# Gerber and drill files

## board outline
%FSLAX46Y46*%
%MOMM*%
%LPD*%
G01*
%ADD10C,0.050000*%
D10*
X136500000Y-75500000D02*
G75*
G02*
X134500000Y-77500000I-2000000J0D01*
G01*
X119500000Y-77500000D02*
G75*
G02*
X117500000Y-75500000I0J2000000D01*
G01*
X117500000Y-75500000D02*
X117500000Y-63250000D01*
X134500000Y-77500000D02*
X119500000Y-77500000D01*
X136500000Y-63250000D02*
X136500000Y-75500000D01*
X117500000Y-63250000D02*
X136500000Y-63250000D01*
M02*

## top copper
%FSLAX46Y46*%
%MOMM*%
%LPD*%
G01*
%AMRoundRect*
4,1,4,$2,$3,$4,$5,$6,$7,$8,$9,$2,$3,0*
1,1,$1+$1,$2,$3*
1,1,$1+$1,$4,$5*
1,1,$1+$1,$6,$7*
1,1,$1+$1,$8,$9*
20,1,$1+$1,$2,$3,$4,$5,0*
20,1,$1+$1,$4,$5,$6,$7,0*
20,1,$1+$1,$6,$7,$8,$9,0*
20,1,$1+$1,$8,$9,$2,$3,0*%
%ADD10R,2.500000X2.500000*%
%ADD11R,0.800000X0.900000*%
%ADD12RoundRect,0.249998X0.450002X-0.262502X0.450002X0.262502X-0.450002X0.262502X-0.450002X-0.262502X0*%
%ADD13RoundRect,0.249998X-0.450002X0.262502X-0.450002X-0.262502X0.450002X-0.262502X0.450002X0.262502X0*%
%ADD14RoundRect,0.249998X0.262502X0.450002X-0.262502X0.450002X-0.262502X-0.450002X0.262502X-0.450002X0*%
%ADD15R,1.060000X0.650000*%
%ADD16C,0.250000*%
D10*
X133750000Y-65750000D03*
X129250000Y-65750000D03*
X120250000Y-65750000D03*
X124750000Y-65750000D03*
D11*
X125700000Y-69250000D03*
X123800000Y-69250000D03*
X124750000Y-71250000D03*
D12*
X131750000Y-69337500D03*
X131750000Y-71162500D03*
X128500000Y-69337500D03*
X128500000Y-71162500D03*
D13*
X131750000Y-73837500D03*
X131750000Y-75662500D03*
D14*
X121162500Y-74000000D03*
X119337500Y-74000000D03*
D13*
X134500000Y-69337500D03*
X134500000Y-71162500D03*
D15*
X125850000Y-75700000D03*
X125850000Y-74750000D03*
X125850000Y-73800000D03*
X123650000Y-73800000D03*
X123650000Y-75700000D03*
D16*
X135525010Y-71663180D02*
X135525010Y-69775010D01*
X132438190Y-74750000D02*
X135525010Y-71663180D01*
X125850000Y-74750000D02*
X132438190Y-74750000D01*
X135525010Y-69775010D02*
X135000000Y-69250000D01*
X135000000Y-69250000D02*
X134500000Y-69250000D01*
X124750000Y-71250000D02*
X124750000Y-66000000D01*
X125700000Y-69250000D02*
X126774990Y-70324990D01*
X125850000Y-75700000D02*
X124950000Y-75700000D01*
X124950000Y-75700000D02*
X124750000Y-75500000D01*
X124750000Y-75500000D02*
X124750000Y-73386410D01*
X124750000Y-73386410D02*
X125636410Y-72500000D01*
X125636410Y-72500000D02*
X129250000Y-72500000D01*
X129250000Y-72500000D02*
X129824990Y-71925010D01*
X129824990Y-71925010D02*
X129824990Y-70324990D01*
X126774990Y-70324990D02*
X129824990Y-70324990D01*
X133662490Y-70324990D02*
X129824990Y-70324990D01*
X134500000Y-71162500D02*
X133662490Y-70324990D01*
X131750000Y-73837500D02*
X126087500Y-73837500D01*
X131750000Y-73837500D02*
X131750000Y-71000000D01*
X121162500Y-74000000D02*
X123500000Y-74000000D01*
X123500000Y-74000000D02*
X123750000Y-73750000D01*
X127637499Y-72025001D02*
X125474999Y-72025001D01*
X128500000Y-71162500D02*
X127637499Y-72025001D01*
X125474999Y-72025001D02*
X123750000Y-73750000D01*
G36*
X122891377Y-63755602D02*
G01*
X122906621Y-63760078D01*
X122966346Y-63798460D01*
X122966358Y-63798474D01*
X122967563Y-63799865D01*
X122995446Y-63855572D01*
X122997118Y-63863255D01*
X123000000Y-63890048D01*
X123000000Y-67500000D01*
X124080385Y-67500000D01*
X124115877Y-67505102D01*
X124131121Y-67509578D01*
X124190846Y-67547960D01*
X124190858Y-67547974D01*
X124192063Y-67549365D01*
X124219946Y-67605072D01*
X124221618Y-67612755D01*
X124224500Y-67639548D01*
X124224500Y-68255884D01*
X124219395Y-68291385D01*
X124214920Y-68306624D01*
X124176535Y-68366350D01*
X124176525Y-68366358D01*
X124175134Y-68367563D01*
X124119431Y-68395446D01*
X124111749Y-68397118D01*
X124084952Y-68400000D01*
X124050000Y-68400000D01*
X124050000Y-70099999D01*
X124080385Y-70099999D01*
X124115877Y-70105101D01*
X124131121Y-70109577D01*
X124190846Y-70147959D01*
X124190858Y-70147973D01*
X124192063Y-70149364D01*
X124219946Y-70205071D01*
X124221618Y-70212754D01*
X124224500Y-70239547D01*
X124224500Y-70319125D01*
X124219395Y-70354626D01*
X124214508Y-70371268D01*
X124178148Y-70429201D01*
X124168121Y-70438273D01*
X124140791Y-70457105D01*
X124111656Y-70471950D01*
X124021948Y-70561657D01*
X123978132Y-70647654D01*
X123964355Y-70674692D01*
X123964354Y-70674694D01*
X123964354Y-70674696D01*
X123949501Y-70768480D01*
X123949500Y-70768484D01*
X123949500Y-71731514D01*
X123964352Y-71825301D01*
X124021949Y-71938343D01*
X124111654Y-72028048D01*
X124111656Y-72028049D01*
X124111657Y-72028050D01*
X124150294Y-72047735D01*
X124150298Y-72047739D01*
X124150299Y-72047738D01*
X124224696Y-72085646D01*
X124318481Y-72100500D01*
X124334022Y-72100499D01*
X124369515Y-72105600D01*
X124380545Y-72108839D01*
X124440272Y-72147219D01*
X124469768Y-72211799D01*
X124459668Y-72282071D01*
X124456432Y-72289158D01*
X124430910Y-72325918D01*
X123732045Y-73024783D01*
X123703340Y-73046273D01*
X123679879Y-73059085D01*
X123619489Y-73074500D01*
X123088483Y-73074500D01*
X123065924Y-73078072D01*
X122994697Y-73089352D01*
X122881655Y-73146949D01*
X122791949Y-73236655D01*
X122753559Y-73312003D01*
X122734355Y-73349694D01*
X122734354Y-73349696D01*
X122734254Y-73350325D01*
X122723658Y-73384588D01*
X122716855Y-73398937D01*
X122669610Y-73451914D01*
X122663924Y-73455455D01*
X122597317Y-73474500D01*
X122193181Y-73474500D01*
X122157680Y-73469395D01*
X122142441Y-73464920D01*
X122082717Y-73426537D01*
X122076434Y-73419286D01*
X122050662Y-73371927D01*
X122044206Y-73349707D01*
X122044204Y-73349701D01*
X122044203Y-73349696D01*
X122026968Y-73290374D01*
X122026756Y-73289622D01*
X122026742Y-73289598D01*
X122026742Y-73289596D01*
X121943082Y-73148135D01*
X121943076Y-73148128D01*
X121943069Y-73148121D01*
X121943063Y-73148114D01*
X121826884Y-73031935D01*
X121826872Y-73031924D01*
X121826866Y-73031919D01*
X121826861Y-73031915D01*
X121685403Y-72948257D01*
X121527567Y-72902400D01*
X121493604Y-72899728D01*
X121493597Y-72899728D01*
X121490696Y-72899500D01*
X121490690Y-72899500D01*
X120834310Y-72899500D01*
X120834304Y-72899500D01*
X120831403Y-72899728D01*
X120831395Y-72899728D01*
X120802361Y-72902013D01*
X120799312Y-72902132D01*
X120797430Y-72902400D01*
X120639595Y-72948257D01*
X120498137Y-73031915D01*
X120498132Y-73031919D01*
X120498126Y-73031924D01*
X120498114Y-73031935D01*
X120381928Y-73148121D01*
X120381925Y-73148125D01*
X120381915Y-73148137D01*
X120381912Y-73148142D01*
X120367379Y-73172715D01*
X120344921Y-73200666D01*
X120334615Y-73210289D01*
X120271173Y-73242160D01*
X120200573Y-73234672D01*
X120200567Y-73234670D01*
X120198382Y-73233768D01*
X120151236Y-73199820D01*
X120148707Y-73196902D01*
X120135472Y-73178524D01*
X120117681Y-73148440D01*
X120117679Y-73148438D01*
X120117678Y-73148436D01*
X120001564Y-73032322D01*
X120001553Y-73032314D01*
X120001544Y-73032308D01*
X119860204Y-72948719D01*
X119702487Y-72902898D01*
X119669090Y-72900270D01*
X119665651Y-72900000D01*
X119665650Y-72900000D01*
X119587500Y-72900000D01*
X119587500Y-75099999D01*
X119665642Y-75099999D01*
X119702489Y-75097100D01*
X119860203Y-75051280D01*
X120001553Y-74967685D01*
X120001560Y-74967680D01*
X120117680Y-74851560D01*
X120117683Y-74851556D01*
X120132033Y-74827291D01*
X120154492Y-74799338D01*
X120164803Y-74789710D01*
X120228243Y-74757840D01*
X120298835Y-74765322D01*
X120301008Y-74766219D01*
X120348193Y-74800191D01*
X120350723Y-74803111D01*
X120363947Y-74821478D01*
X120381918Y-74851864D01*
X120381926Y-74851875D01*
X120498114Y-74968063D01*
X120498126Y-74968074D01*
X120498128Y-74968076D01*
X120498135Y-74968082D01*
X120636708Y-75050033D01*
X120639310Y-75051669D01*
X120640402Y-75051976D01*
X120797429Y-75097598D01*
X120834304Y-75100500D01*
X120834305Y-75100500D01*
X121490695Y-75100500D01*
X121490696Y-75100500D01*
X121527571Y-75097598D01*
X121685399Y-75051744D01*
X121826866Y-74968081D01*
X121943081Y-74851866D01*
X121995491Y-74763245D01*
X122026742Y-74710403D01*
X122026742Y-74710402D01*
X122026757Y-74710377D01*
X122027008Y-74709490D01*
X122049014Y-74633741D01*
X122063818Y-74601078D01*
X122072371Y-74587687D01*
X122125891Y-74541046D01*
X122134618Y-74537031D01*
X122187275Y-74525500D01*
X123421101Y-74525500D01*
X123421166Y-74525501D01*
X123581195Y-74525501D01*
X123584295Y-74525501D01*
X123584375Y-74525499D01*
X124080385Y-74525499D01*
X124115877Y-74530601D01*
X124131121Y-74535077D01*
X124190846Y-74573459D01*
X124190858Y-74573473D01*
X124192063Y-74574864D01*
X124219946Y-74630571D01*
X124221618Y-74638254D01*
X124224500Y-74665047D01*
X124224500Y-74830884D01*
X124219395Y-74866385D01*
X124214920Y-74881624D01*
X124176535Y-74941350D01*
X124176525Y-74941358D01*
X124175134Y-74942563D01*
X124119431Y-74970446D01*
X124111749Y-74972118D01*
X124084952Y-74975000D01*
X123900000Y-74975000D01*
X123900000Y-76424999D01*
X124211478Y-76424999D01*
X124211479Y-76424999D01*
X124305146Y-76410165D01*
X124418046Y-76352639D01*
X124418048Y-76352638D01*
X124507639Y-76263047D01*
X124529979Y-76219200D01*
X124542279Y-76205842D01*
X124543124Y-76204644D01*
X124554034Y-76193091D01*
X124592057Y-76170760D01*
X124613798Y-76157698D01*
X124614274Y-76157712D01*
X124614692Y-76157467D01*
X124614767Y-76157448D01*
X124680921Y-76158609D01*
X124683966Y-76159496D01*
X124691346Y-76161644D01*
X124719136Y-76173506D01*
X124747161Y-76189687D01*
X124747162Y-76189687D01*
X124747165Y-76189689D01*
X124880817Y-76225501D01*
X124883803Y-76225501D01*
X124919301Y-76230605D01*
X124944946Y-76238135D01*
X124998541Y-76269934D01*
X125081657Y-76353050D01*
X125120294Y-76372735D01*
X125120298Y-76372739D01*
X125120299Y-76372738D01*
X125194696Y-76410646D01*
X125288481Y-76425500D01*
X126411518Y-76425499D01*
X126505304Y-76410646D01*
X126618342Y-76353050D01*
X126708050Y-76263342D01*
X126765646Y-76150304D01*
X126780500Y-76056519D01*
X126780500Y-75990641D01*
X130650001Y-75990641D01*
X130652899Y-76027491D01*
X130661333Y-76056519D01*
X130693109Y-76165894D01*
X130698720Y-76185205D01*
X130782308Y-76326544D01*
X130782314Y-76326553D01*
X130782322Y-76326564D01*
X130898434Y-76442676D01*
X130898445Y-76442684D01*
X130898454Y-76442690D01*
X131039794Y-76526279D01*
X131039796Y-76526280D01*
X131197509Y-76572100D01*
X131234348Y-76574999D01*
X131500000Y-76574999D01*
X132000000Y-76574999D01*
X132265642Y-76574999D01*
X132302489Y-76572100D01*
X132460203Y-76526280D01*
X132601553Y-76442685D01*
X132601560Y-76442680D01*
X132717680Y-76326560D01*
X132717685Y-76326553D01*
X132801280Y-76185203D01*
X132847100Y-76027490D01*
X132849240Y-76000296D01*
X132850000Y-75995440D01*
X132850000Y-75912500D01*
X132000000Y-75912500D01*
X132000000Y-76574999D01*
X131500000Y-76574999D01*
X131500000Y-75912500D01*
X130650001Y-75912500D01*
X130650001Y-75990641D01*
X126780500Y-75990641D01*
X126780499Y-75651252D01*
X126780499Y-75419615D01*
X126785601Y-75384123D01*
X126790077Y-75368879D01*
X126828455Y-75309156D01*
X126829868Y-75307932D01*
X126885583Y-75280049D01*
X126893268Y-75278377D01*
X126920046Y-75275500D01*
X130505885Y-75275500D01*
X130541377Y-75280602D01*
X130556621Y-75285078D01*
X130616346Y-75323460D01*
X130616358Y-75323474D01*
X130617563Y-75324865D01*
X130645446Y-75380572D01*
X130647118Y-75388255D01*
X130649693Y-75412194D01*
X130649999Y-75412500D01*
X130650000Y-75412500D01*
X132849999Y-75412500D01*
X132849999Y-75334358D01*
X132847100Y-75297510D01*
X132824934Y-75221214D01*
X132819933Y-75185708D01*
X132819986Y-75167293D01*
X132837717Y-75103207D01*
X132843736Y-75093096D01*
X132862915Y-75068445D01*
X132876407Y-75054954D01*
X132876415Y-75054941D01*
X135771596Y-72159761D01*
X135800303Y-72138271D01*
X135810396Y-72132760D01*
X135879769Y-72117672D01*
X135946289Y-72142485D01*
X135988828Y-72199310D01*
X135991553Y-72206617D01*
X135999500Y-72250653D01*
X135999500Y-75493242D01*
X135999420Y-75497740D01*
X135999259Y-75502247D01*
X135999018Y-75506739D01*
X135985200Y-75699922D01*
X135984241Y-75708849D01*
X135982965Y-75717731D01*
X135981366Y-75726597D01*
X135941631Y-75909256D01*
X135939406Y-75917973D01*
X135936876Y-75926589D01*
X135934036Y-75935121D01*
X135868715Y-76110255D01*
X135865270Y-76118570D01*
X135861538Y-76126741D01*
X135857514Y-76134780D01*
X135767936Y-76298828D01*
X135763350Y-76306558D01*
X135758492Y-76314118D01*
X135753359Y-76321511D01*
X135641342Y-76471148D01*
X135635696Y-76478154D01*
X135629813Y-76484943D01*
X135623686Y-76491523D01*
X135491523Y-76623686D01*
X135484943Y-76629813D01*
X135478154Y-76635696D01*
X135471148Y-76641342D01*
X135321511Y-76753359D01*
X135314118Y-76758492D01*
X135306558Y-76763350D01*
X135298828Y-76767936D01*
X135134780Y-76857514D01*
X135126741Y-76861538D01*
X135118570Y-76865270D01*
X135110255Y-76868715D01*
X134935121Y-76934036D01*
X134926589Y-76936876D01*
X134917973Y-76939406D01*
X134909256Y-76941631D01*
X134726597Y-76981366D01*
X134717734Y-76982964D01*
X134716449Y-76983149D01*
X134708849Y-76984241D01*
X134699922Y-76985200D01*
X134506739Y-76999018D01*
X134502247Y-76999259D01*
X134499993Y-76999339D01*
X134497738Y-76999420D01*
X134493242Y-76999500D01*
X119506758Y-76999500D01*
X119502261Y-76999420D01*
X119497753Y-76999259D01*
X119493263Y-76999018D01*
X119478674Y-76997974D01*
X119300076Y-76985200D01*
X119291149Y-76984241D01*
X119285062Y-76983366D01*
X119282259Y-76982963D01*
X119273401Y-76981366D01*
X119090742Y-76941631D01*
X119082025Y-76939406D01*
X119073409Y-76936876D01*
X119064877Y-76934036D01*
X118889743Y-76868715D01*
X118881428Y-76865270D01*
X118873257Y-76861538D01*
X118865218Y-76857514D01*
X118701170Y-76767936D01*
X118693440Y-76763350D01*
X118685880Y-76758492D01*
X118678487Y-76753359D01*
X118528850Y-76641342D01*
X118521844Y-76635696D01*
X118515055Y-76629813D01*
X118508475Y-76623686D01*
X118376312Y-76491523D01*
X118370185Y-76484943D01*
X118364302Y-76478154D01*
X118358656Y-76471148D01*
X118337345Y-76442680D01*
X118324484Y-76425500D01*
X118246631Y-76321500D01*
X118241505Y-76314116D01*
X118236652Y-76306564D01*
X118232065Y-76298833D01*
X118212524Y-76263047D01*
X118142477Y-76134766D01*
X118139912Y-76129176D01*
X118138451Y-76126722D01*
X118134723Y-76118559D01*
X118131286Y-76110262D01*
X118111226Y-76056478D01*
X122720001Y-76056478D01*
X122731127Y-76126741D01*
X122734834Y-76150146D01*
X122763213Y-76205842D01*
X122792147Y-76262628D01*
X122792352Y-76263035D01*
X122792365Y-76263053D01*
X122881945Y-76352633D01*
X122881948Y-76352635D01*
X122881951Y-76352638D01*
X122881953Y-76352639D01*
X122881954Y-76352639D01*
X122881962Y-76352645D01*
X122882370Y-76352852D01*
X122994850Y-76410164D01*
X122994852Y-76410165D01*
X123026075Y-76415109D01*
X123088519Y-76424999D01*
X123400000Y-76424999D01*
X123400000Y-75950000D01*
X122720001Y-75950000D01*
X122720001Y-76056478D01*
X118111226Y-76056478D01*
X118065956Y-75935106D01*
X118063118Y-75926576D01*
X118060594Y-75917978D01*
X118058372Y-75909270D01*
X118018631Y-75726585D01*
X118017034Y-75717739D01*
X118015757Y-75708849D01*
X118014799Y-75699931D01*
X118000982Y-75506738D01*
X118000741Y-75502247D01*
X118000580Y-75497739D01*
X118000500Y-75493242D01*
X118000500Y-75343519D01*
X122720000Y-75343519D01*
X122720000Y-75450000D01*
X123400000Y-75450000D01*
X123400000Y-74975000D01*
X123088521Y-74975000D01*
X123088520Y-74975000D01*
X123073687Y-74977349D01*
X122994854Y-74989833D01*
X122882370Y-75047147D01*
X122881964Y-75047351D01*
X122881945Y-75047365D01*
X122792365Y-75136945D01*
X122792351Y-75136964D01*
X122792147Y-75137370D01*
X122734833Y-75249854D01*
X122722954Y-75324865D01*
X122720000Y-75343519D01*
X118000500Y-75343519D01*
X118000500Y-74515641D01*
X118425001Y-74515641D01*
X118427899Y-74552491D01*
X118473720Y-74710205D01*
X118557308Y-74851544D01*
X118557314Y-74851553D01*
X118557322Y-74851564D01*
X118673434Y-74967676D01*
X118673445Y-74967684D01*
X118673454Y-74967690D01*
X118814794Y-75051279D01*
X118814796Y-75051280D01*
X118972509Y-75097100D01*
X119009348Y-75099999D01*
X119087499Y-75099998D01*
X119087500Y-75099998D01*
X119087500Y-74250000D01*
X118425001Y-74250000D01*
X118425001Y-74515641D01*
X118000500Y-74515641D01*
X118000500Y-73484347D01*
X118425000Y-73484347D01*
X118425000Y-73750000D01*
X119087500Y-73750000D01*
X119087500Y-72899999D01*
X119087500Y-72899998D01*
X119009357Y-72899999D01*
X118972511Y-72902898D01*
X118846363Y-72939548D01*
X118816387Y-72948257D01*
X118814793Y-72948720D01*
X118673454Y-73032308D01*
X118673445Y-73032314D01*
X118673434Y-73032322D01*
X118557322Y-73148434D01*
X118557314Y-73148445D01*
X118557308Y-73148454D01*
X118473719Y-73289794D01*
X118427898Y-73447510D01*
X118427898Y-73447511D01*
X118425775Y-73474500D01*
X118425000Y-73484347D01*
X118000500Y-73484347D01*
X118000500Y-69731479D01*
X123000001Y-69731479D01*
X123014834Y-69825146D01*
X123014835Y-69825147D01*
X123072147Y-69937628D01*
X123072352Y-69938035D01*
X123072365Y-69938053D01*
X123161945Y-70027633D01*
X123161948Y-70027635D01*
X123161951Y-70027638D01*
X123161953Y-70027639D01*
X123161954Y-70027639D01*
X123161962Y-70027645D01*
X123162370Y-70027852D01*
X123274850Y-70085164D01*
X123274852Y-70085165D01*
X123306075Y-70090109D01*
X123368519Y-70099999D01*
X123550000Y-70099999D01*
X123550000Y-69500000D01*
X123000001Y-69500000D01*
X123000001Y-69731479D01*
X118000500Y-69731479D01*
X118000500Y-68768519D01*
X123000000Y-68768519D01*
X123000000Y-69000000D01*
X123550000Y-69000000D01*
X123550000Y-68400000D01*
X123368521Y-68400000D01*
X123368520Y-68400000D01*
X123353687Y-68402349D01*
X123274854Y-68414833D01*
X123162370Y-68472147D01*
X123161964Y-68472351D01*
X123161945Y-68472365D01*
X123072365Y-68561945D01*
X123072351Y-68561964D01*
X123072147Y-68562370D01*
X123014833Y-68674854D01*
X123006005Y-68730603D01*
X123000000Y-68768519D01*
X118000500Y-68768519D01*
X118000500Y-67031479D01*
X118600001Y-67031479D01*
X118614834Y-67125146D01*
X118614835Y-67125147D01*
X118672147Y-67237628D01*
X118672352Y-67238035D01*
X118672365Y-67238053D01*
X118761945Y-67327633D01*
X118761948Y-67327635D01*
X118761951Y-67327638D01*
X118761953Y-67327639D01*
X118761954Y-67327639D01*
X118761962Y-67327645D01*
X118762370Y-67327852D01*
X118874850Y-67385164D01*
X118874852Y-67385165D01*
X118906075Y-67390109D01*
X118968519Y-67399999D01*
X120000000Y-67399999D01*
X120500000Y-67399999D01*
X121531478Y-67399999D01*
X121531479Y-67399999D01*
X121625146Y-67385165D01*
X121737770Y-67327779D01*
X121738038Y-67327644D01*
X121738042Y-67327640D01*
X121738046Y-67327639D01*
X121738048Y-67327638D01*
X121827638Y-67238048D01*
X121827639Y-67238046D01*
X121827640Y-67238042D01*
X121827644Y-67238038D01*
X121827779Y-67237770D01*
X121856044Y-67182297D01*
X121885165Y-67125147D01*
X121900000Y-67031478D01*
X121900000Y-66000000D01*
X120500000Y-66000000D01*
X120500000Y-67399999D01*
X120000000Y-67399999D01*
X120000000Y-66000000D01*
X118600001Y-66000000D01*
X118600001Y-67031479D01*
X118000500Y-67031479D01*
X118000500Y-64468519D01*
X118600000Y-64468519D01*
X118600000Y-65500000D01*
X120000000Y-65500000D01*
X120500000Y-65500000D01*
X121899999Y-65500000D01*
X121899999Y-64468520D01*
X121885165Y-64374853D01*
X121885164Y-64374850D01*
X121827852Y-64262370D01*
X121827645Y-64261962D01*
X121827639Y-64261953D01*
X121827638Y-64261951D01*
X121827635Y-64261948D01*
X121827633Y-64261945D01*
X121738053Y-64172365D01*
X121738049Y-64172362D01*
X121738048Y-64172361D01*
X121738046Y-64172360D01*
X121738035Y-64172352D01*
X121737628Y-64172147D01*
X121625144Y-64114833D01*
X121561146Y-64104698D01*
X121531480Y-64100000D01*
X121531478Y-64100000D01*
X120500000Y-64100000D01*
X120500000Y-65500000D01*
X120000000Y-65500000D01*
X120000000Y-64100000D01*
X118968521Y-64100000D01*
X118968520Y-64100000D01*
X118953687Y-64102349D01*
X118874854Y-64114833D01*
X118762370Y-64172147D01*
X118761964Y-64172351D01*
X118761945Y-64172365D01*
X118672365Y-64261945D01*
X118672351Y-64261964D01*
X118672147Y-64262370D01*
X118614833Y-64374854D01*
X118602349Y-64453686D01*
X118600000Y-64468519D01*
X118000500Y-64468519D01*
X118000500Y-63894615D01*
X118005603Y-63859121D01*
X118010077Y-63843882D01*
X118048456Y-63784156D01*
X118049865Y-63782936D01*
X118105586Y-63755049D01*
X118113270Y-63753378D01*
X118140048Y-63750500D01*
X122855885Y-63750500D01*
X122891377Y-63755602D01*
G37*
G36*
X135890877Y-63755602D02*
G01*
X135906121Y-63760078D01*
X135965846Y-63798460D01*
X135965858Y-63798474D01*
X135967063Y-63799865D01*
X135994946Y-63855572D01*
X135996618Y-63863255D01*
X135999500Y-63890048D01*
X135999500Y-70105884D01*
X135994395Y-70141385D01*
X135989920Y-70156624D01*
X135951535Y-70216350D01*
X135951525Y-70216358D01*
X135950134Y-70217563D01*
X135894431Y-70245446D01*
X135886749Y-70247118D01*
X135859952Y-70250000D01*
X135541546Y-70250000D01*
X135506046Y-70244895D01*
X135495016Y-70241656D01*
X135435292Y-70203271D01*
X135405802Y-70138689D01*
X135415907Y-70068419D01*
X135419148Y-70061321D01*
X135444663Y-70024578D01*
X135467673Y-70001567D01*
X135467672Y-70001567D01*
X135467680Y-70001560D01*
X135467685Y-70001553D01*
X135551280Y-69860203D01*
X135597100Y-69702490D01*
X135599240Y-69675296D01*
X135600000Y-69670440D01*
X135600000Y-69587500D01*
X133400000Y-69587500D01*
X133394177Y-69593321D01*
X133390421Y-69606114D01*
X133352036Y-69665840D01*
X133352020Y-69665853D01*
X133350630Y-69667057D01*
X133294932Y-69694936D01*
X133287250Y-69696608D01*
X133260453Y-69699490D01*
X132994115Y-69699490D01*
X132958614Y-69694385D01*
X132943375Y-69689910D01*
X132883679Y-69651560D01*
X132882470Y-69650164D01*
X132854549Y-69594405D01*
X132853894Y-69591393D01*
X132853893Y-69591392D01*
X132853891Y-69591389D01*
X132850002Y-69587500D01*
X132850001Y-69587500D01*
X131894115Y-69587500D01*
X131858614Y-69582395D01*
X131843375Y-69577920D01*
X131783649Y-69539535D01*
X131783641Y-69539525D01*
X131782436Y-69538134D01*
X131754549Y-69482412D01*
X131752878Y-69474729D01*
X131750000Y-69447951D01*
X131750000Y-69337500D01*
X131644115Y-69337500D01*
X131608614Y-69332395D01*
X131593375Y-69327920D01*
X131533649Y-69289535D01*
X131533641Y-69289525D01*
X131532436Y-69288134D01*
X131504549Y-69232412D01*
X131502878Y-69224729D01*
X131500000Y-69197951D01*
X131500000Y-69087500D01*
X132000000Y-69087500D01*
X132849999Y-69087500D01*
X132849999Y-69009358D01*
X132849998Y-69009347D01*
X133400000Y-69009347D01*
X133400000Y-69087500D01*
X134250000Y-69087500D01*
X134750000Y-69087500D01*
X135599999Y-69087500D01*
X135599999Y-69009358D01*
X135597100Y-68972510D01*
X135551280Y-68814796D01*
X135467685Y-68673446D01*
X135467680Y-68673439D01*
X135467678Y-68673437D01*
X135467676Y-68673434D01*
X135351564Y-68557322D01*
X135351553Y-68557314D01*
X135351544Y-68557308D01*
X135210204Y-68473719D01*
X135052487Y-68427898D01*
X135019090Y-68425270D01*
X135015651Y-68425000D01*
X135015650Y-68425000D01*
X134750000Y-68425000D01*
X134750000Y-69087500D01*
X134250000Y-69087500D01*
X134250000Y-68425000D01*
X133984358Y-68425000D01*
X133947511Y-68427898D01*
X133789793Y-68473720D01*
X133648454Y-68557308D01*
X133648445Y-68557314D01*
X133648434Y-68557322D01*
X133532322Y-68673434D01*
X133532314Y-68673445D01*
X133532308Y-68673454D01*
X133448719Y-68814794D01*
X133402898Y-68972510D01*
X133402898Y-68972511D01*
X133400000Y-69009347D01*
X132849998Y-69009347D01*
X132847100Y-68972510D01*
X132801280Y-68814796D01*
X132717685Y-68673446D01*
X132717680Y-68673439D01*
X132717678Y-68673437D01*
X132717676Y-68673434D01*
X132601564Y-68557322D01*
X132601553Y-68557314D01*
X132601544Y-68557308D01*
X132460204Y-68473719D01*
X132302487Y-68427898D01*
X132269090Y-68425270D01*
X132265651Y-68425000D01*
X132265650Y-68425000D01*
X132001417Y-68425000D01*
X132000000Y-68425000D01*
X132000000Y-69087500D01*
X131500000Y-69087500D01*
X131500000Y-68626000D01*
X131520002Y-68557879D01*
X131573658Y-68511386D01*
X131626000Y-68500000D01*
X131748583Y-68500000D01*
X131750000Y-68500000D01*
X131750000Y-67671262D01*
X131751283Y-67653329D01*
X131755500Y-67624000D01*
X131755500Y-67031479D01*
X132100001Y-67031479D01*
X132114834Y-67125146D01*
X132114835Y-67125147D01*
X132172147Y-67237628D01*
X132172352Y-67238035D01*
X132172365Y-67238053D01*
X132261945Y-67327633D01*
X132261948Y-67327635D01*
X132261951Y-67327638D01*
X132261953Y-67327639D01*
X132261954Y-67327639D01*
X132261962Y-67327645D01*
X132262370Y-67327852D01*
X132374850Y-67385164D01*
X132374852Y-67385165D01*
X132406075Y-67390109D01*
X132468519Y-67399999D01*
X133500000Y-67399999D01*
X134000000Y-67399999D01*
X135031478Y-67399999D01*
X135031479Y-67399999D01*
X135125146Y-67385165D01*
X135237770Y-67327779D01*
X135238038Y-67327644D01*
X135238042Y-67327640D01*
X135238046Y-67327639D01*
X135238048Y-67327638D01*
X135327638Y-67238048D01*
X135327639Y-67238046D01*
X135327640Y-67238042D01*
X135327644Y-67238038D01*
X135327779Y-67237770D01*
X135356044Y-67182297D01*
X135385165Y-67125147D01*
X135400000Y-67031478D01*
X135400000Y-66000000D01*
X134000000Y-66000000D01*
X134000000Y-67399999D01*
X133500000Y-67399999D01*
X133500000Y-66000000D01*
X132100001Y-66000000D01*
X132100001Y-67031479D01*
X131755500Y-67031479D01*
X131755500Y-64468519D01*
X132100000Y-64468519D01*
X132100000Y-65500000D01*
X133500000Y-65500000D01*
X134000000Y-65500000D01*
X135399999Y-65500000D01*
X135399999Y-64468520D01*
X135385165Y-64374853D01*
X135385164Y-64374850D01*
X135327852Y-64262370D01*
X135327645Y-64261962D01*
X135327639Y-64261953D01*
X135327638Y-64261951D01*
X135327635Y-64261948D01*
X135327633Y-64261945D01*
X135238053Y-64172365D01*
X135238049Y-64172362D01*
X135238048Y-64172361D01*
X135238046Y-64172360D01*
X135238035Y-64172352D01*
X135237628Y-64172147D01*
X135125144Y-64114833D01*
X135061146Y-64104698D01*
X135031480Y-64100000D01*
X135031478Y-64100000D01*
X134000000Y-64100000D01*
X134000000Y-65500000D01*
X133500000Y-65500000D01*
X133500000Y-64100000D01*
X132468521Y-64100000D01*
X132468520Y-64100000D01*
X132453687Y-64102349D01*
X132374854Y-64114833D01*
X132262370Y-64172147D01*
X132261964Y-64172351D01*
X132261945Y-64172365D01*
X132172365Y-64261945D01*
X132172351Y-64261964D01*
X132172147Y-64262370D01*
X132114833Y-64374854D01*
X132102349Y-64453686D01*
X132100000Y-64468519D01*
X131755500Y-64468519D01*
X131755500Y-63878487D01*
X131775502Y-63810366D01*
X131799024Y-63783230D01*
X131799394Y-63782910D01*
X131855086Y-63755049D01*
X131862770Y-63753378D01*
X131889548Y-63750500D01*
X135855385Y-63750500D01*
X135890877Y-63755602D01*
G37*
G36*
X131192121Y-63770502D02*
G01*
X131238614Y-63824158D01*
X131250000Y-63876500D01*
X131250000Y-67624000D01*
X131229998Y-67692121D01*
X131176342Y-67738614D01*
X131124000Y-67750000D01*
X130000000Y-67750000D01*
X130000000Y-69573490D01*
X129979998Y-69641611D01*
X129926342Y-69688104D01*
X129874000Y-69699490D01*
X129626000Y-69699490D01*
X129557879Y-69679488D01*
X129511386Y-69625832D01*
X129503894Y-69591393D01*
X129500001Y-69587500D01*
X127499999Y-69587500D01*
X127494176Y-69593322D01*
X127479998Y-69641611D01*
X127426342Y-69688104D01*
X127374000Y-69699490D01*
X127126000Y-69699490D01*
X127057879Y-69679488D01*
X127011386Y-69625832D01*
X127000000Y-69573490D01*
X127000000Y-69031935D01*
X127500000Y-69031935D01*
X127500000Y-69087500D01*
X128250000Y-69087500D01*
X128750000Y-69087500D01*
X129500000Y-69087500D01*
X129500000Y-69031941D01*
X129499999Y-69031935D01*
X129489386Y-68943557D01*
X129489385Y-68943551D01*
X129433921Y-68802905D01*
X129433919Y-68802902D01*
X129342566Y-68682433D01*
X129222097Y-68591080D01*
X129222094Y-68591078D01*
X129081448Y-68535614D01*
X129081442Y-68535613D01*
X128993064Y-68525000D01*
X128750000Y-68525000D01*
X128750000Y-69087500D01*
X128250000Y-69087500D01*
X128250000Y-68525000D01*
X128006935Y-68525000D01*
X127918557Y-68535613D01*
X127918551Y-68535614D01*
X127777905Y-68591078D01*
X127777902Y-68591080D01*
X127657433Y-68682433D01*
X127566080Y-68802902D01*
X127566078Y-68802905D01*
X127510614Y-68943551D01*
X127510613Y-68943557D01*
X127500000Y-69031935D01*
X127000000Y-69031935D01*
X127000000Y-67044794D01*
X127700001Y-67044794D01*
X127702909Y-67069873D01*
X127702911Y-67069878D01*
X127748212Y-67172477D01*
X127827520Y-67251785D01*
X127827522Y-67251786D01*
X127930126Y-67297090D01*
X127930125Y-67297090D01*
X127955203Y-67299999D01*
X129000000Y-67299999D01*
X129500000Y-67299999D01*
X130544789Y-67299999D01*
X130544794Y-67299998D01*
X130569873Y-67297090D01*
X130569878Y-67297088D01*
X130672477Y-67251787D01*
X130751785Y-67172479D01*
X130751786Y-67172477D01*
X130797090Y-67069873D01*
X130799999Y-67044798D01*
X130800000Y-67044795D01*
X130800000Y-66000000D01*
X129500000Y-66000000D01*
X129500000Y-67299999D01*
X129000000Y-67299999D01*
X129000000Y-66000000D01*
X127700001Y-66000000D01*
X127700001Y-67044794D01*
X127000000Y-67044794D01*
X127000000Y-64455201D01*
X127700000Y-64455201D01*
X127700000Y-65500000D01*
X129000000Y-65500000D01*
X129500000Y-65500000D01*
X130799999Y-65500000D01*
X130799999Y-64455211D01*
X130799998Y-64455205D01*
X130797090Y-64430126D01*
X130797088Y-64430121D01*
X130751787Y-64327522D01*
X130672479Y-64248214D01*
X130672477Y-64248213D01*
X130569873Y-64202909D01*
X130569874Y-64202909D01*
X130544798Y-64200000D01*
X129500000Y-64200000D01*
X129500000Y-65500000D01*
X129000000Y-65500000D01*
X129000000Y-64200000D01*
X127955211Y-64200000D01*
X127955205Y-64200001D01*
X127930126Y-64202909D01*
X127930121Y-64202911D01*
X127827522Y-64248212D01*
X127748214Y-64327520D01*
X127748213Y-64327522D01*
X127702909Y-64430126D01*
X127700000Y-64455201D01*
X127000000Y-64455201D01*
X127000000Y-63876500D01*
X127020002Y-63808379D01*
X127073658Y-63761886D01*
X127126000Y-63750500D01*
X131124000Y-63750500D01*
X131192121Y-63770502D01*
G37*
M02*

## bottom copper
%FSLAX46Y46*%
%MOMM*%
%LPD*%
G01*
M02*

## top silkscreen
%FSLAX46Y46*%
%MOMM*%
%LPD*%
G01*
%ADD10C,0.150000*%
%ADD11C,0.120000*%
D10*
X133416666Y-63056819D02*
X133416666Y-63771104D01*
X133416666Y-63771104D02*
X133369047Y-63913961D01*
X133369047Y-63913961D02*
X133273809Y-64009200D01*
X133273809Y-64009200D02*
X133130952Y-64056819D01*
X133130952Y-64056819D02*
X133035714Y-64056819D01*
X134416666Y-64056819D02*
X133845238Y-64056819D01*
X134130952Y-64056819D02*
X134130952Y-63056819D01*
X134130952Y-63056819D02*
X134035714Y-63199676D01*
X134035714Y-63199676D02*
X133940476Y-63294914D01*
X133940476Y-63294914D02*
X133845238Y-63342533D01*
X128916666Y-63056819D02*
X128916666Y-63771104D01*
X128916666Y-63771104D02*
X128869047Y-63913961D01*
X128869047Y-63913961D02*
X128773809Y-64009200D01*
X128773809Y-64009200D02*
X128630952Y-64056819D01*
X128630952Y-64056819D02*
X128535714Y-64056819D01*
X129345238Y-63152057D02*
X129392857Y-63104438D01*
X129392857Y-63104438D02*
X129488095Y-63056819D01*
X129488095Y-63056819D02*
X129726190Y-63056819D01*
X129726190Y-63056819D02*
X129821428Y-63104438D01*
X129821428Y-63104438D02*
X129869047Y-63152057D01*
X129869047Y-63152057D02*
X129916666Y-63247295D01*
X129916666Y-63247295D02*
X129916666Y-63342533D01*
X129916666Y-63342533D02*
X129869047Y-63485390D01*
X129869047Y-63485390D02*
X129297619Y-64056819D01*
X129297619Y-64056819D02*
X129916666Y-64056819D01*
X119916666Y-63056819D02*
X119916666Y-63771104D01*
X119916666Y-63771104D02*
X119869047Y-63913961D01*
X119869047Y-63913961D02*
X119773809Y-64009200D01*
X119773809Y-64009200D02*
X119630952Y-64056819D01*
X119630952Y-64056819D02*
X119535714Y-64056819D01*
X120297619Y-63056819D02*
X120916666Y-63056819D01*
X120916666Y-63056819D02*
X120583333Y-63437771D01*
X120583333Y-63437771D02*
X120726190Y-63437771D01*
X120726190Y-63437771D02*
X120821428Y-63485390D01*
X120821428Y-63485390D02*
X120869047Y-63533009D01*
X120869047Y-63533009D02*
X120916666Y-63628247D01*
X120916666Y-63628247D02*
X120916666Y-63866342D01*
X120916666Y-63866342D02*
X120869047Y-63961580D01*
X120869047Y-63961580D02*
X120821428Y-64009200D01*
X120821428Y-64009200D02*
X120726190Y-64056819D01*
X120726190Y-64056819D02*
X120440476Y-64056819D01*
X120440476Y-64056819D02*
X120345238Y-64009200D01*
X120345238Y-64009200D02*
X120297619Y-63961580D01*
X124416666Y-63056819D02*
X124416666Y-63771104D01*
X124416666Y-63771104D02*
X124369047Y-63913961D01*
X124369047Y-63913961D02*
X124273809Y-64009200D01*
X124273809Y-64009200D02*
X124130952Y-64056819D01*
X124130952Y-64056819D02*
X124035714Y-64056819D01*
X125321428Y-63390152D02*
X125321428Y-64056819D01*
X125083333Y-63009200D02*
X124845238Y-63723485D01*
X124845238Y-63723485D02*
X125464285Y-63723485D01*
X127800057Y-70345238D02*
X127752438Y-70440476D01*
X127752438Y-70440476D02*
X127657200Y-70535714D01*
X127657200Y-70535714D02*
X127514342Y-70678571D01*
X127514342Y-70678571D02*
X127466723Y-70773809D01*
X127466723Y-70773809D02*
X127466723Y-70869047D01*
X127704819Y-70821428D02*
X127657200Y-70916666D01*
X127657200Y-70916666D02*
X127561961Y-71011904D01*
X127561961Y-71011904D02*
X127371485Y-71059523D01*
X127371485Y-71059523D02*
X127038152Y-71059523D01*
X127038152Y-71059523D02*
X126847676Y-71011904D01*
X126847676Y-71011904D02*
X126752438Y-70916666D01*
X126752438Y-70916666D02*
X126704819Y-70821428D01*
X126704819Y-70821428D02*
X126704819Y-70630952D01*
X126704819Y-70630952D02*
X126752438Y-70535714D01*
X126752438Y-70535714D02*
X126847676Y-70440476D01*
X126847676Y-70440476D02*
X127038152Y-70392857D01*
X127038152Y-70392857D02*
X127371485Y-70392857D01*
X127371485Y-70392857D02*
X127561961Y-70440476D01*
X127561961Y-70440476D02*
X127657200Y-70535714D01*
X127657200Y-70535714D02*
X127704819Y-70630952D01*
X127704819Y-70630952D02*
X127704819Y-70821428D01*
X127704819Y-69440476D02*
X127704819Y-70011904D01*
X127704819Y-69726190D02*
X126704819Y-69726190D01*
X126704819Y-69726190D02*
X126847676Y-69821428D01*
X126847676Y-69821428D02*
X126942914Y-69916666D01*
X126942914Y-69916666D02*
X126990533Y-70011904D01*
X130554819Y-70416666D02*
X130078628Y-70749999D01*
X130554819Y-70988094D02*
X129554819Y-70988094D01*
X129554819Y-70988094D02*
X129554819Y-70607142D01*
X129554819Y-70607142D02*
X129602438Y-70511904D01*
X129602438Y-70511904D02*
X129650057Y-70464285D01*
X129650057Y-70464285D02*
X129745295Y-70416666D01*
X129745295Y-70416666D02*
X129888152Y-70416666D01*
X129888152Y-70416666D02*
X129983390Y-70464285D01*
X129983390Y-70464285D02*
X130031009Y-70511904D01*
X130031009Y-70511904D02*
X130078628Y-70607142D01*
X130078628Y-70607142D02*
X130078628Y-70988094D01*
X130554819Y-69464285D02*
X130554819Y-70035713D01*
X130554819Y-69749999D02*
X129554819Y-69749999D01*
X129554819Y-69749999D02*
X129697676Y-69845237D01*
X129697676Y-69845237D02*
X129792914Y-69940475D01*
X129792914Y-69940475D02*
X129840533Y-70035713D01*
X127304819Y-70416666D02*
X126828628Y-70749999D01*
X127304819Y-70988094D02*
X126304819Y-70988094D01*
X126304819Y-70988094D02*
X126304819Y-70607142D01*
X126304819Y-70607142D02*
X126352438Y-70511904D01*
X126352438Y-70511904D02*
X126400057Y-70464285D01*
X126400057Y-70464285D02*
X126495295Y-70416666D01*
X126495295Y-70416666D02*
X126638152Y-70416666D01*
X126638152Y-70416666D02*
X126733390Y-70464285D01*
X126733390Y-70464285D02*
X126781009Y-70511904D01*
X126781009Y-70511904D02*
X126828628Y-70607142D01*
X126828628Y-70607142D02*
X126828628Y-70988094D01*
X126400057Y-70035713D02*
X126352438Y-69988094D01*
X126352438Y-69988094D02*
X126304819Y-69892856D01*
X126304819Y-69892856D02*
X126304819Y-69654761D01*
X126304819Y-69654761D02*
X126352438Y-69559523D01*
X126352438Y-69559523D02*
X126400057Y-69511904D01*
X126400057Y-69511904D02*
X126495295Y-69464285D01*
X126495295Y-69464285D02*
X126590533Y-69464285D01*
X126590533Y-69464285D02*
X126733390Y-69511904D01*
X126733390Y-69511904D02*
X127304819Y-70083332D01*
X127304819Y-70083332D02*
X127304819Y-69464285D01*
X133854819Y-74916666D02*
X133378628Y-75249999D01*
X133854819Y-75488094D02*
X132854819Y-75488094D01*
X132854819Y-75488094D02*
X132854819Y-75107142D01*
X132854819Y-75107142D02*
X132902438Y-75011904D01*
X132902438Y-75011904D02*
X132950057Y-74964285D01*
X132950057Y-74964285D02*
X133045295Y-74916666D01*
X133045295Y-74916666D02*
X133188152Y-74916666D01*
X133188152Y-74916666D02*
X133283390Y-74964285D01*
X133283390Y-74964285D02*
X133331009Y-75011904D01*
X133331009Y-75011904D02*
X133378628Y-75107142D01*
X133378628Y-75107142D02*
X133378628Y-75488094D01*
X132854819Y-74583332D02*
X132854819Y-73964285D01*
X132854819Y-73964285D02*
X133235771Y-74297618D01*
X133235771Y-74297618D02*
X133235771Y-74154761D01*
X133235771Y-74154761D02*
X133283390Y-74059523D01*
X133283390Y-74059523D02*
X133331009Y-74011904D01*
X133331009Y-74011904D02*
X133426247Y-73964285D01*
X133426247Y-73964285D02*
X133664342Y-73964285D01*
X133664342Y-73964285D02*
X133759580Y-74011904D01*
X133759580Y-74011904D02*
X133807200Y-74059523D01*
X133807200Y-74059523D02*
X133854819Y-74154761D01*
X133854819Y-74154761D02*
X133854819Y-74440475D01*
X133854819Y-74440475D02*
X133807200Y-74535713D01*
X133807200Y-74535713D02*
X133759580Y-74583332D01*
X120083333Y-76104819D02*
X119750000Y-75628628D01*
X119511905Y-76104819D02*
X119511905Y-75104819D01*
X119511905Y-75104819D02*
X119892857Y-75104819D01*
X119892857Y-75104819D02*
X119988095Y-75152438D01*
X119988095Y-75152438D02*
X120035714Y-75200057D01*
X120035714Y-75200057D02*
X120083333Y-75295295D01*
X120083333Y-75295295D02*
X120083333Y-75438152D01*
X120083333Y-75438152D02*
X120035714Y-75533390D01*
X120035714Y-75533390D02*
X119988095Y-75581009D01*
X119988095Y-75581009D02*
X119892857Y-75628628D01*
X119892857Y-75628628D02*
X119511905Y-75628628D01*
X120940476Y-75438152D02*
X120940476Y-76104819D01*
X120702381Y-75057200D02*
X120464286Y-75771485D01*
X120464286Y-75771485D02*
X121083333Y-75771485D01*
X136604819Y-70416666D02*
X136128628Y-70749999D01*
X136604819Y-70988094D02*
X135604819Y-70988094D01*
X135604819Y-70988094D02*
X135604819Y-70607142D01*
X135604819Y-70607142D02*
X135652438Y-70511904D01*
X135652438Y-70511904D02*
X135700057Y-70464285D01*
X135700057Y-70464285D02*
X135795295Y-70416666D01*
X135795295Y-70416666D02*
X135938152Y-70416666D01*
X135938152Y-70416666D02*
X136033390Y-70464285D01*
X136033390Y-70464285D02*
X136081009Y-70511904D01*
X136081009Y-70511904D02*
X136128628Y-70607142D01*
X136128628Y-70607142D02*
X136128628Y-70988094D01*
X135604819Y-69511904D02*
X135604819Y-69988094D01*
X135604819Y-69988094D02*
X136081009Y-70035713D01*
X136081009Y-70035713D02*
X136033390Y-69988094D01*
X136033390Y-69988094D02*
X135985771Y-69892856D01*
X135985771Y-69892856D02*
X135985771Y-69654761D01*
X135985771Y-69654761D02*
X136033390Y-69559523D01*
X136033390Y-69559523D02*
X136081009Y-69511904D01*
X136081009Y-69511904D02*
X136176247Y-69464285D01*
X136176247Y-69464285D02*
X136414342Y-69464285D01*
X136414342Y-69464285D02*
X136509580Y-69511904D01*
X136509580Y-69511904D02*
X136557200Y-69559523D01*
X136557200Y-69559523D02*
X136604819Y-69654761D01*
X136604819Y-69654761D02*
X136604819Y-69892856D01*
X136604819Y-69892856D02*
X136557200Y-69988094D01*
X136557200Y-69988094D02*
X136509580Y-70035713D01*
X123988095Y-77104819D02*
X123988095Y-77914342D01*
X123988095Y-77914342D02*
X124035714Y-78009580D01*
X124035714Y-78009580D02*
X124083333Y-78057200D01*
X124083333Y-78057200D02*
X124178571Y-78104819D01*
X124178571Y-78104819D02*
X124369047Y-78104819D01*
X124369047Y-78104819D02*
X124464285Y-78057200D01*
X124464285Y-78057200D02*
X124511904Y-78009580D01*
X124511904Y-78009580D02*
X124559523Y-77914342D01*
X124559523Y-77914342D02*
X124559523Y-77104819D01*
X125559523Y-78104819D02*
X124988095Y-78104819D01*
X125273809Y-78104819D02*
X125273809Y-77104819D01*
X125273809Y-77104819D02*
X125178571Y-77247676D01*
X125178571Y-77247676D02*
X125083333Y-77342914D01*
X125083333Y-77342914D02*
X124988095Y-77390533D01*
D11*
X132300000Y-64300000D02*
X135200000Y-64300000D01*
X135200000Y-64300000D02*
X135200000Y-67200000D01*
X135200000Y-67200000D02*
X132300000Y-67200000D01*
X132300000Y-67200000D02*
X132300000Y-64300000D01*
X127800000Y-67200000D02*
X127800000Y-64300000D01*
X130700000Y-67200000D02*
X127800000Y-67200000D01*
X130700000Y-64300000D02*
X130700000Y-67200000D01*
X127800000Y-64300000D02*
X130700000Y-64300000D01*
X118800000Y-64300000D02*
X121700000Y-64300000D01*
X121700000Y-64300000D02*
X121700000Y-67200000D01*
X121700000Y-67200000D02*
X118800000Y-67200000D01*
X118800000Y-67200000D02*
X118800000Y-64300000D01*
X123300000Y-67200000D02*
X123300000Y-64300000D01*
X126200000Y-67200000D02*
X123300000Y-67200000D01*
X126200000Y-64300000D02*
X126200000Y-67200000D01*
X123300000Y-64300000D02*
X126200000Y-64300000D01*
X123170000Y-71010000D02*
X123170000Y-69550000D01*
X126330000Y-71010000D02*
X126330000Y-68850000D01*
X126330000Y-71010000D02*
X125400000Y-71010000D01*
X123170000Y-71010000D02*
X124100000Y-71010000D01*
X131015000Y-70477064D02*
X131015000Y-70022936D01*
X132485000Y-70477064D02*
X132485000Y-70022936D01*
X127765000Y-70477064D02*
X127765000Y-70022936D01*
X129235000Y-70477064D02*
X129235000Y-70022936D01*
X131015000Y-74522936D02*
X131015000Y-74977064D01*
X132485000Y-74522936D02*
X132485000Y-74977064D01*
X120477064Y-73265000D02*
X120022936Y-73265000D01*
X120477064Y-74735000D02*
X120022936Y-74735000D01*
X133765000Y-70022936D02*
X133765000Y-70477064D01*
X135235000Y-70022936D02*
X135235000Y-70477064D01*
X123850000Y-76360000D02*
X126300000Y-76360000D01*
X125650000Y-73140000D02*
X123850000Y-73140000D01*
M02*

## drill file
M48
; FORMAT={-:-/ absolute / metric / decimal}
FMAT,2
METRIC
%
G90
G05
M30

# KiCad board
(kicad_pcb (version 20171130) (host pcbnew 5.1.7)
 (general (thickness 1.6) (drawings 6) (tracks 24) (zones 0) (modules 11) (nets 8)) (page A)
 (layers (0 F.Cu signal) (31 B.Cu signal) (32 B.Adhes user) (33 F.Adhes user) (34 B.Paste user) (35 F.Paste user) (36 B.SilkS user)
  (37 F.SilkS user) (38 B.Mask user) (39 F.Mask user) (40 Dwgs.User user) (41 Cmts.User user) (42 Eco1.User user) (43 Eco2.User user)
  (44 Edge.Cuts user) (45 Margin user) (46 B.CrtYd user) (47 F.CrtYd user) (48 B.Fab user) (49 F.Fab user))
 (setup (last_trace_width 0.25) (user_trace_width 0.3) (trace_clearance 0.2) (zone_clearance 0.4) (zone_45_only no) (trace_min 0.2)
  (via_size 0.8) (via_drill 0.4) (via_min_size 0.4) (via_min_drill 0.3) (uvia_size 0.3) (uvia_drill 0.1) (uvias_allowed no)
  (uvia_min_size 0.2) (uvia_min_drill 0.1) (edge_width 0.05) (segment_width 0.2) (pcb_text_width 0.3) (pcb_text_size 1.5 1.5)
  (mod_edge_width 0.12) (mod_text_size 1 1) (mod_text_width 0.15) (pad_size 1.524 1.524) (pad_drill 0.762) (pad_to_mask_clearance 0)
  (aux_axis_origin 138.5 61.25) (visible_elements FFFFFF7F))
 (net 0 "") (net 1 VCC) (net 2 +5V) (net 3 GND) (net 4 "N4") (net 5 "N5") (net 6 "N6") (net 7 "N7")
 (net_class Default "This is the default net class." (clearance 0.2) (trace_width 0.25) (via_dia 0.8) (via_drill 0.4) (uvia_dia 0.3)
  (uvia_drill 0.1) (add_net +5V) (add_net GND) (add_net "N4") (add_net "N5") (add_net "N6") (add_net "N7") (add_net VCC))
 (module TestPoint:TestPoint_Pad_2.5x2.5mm (layer F.Cu) (at 133.75 65.75)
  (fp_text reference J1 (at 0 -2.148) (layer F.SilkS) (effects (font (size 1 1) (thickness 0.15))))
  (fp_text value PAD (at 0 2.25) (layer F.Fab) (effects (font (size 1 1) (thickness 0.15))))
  (fp_line (start -1.45 -1.45) (end 1.45 -1.45) (layer F.SilkS) (width 0.12))
  (fp_line (start 1.45 -1.45) (end 1.45 1.45) (layer F.SilkS) (width 0.12))
  (fp_line (start 1.45 1.45) (end -1.45 1.45) (layer F.SilkS) (width 0.12))
  (fp_line (start -1.45 1.45) (end -1.45 -1.45) (layer F.SilkS) (width 0.12))
  (pad 1 smd rect (at 0 0) (size 2.5 2.5) (layers F.Cu F.Mask) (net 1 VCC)))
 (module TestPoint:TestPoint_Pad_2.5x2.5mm (layer F.Cu) (at 129.25 65.75)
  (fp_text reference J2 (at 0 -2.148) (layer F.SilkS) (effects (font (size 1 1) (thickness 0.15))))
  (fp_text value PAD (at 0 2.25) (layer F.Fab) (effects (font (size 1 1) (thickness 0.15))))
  (fp_line (start -1.45 1.45) (end -1.45 -1.45) (layer F.SilkS) (width 0.12))
  (fp_line (start 1.45 1.45) (end -1.45 1.45) (layer F.SilkS) (width 0.12))
  (fp_line (start 1.45 -1.45) (end 1.45 1.45) (layer F.SilkS) (width 0.12))
  (fp_line (start -1.45 -1.45) (end 1.45 -1.45) (layer F.SilkS) (width 0.12))
  (pad 1 smd rect (at 0 0) (size 2.5 2.5) (layers F.Cu F.Mask) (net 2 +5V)))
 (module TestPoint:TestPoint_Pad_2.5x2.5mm (layer F.Cu) (at 120.25 65.75)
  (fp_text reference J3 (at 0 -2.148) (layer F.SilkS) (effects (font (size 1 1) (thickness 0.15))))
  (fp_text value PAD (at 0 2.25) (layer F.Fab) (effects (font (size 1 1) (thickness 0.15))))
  (fp_line (start -1.45 -1.45) (end 1.45 -1.45) (layer F.SilkS) (width 0.12))
  (fp_line (start 1.45 -1.45) (end 1.45 1.45) (layer F.SilkS) (width 0.12))
  (fp_line (start 1.45 1.45) (end -1.45 1.45) (layer F.SilkS) (width 0.12))
  (fp_line (start -1.45 1.45) (end -1.45 -1.45) (layer F.SilkS) (width 0.12))
  (pad 1 smd rect (at 0 0) (size 2.5 2.5) (layers F.Cu F.Mask) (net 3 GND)))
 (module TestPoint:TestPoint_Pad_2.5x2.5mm (layer F.Cu) (at 124.75 65.75)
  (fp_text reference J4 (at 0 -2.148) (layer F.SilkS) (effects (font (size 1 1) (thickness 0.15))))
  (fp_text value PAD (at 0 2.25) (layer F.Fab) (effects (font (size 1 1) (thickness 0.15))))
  (fp_line (start -1.45 1.45) (end -1.45 -1.45) (layer F.SilkS) (width 0.12))
  (fp_line (start 1.45 1.45) (end -1.45 1.45) (layer F.SilkS) (width 0.12))
  (fp_line (start 1.45 -1.45) (end 1.45 1.45) (layer F.SilkS) (width 0.12))
  (fp_line (start -1.45 -1.45) (end 1.45 -1.45) (layer F.SilkS) (width 0.12))
  (pad 1 smd rect (at 0 0) (size 2.5 2.5) (layers F.Cu F.Mask) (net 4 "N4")))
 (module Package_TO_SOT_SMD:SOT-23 (layer F.Cu) (at 124.75 70.25 270)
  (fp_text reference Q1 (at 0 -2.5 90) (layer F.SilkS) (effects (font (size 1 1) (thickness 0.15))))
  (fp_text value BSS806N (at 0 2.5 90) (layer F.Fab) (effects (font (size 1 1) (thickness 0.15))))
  (fp_line (start 0.76 1.58) (end -0.7 1.58) (layer F.SilkS) (width 0.12))
  (fp_line (start 0.76 -1.58) (end -1.4 -1.58) (layer F.SilkS) (width 0.12))
  (fp_line (start 0.76 -1.58) (end 0.76 -0.65) (layer F.SilkS) (width 0.12))
  (fp_line (start 0.76 1.58) (end 0.76 0.65) (layer F.SilkS) (width 0.12))
  (pad 1 smd rect (at -1 -0.95 270) (size 0.9 0.8) (layers F.Cu F.Paste F.Mask) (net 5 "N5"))
  (pad 2 smd rect (at -1 0.95 270) (size 0.9 0.8) (layers F.Cu F.Paste F.Mask) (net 3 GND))
  (pad 3 smd rect (at 1 0 270) (size 0.9 0.8) (layers F.Cu F.Paste F.Mask) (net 4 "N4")))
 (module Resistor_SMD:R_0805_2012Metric (layer F.Cu) (at 131.75 70.25 90)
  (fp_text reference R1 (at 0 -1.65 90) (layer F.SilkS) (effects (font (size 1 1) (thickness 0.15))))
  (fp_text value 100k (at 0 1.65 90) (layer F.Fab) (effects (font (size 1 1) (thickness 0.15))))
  (fp_line (start -0.227064 -0.735) (end 0.227064 -0.735) (layer F.SilkS) (width 0.12))
  (fp_line (start -0.227064 0.735) (end 0.227064 0.735) (layer F.SilkS) (width 0.12))
  (pad 2 smd roundrect (at 0.9125 0 90) (size 1.025 1.4) (layers F.Cu F.Paste F.Mask) (roundrect_rratio 0.2439004878048781) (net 1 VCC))
  (pad 1 smd roundrect (at -0.9125 0 90) (size 1.025 1.4) (layers F.Cu F.Paste F.Mask) (roundrect_rratio 0.2439004878048781) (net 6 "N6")))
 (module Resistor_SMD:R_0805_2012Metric (layer F.Cu) (at 128.5 70.25 90)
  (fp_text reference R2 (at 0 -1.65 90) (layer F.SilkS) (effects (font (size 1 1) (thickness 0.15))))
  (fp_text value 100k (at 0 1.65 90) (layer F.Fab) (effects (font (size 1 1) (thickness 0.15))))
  (fp_line (start -0.227064 -0.735) (end 0.227064 -0.735) (layer F.SilkS) (width 0.12))
  (fp_line (start -0.227064 0.735) (end 0.227064 0.735) (layer F.SilkS) (width 0.12))
  (pad 2 smd roundrect (at 0.9125 0 90) (size 1.025 1.4) (layers F.Cu F.Paste F.Mask) (roundrect_rratio 0.2439004878048781) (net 2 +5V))
  (pad 1 smd roundrect (at -0.9125 0 90) (size 1.025 1.4) (layers F.Cu F.Paste F.Mask) (roundrect_rratio 0.2439004878048781) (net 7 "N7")))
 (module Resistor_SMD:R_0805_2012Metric (layer F.Cu) (at 131.75 74.75 270)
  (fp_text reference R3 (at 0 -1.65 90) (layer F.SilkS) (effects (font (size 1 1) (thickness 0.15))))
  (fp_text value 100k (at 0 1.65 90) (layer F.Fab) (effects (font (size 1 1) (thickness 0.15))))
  (fp_line (start -0.227064 0.735) (end 0.227064 0.735) (layer F.SilkS) (width 0.12))
  (fp_line (start -0.227064 -0.735) (end 0.227064 -0.735) (layer F.SilkS) (width 0.12))
  (pad 1 smd roundrect (at -0.9125 0 270) (size 1.025 1.4) (layers F.Cu F.Paste F.Mask) (roundrect_rratio 0.2439004878048781) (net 6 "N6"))
  (pad 2 smd roundrect (at 0.9125 0 270) (size 1.025 1.4) (layers F.Cu F.Paste F.Mask) (roundrect_rratio 0.2439004878048781) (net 3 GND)))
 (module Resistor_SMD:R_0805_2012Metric (layer F.Cu) (at 120.25 74 180)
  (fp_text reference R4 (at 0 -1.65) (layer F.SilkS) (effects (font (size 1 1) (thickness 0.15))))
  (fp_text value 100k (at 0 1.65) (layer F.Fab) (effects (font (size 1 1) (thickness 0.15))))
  (fp_line (start -0.227064 0.735) (end 0.227064 0.735) (layer F.SilkS) (width 0.12))
  (fp_line (start -0.227064 -0.735) (end 0.227064 -0.735) (layer F.SilkS) (width 0.12))
  (pad 1 smd roundrect (at -0.9125 0 180) (size 1.025 1.4) (layers F.Cu F.Paste F.Mask) (roundrect_rratio 0.2439004878048781) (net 7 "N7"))
  (pad 2 smd roundrect (at 0.9125 0 180) (size 1.025 1.4) (layers F.Cu F.Paste F.Mask) (roundrect_rratio 0.2439004878048781) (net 3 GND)))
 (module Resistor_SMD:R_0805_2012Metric (layer F.Cu) (at 134.5 70.25 270)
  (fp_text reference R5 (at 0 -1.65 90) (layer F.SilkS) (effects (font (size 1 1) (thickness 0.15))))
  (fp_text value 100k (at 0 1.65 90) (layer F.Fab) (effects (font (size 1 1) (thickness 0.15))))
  (fp_line (start -0.227064 0.735) (end 0.227064 0.735) (layer F.SilkS) (width 0.12))
  (fp_line (start -0.227064 -0.735) (end 0.227064 -0.735) (layer F.SilkS) (width 0.12))
  (pad 1 smd roundrect (at -0.9125 0 270) (size 1.025 1.4) (layers F.Cu F.Paste F.Mask) (roundrect_rratio 0.2439004878048781) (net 1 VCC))
  (pad 2 smd roundrect (at 0.9125 0 270) (size 1.025 1.4) (layers F.Cu F.Paste F.Mask) (roundrect_rratio 0.2439004878048781) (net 5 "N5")))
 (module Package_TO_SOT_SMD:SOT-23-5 (layer F.Cu) (at 124.75 74.75 180)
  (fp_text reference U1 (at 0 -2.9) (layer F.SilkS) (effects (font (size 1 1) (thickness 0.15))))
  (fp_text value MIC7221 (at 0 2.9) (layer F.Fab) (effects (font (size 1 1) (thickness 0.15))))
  (fp_line (start 0.9 -1.61) (end -1.55 -1.61) (layer F.SilkS) (width 0.12))
  (fp_line (start -0.9 1.61) (end 0.9 1.61) (layer F.SilkS) (width 0.12))
  (pad 1 smd rect (at -1.1 -0.95 180) (size 1.06 0.65) (layers F.Cu F.Paste F.Mask) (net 5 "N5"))
  (pad 2 smd rect (at -1.1 0 180) (size 1.06 0.65) (layers F.Cu F.Paste F.Mask) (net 1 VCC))
  (pad 3 smd rect (at -1.1 0.95 180) (size 1.06 0.65) (layers F.Cu F.Paste F.Mask) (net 6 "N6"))
  (pad 4 smd rect (at 1.1 0.95 180) (size 1.06 0.65) (layers F.Cu F.Paste F.Mask) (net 7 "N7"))
  (pad 5 smd rect (at 1.1 -0.95 180) (size 1.06 0.65) (layers F.Cu F.Paste F.Mask) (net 3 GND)))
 (gr_arc (start 134.5 75.5) (end 134.5 77.5) (angle -90) (layer Edge.Cuts) (width 0.05))
 (gr_arc (start 119.5 75.5) (end 117.5 75.5) (angle -90) (layer Edge.Cuts) (width 0.05))
 (gr_line (start 117.5 75.5) (end 117.5 63.25) (layer Edge.Cuts) (width 0.05))
 (gr_line (start 134.5 77.5) (end 119.5 77.5) (layer Edge.Cuts) (width 0.05))
 (gr_line (start 136.5 63.25) (end 136.5 75.5) (layer Edge.Cuts) (width 0.05))
 (gr_line (start 117.5 63.25) (end 136.5 63.25) (layer Edge.Cuts) (width 0.05))
 (segment (start 135.52501 71.66318) (end 135.52501 69.77501) (width 0.25) (layer F.Cu) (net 1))
 (segment (start 132.43819 74.75) (end 135.52501 71.66318) (width 0.25) (layer F.Cu) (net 1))
 (segment (start 125.85 74.75) (end 132.43819 74.75) (width 0.25) (layer F.Cu) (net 1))
 (segment (start 135.52501 69.77501) (end 135 69.25) (width 0.25) (layer F.Cu) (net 1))
 (segment (start 135 69.25) (end 134.5 69.25) (width 0.25) (layer F.Cu) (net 1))
 (segment (start 124.75 71.25) (end 124.75 66) (width 0.25) (layer F.Cu) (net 4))
 (segment (start 125.7 69.25) (end 126.77499 70.32499) (width 0.25) (layer F.Cu) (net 5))
 (segment (start 125.85 75.7) (end 124.95 75.7) (width 0.25) (layer F.Cu) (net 5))
 (segment (start 124.95 75.7) (end 124.75 75.5) (width 0.25) (layer F.Cu) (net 5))
 (segment (start 124.75 75.5) (end 124.75 73.38641) (width 0.25) (layer F.Cu) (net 5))
 (segment (start 124.75 73.38641) (end 125.63641 72.5) (width 0.25) (layer F.Cu) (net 5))
 (segment (start 125.63641 72.5) (end 129.25 72.5) (width 0.25) (layer F.Cu) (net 5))
 (segment (start 129.25 72.5) (end 129.82499 71.92501) (width 0.25) (layer F.Cu) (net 5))
 (segment (start 129.82499 71.92501) (end 129.82499 70.32499) (width 0.25) (layer F.Cu) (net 5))
 (segment (start 126.77499 70.32499) (end 129.82499 70.32499) (width 0.25) (layer F.Cu) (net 5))
 (segment (start 133.66249 70.32499) (end 129.82499 70.32499) (width 0.25) (layer F.Cu) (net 5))
 (segment (start 134.5 71.1625) (end 133.66249 70.32499) (width 0.25) (layer F.Cu) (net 5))
 (segment (start 131.75 73.8375) (end 126.0875 73.8375) (width 0.25) (layer F.Cu) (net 6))
 (segment (start 131.75 73.8375) (end 131.75 71) (width 0.25) (layer F.Cu) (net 6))
 (segment (start 121.1625 74) (end 123.5 74) (width 0.25) (layer F.Cu) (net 7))
 (segment (start 123.5 74) (end 123.75 73.75) (width 0.25) (layer F.Cu) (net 7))
 (segment (start 127.637499 72.025001) (end 125.474999 72.025001) (width 0.25) (layer F.Cu) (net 7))
 (segment (start 128.5 71.1625) (end 127.637499 72.025001) (width 0.25) (layer F.Cu) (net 7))
 (segment (start 125.474999 72.025001) (end 123.75 73.75) (width 0.25) (layer F.Cu) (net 7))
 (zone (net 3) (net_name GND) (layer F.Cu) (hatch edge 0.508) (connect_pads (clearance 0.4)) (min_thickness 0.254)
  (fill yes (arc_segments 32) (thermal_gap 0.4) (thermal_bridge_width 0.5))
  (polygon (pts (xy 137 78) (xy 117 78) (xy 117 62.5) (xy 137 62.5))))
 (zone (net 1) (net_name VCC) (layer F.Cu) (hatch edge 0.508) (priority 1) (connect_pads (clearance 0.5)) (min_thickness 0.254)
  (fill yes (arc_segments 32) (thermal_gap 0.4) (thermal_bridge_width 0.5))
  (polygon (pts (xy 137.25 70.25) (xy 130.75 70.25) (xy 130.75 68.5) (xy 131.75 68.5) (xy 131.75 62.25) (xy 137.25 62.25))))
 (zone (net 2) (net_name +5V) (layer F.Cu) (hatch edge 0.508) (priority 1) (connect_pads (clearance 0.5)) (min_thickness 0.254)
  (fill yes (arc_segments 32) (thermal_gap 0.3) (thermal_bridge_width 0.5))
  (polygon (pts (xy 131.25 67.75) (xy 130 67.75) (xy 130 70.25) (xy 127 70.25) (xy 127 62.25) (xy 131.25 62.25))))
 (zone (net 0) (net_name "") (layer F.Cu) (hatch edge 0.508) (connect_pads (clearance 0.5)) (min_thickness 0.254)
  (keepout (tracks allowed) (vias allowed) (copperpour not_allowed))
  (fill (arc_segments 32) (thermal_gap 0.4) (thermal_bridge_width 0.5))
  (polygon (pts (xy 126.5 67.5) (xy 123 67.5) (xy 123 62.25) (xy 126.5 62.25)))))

